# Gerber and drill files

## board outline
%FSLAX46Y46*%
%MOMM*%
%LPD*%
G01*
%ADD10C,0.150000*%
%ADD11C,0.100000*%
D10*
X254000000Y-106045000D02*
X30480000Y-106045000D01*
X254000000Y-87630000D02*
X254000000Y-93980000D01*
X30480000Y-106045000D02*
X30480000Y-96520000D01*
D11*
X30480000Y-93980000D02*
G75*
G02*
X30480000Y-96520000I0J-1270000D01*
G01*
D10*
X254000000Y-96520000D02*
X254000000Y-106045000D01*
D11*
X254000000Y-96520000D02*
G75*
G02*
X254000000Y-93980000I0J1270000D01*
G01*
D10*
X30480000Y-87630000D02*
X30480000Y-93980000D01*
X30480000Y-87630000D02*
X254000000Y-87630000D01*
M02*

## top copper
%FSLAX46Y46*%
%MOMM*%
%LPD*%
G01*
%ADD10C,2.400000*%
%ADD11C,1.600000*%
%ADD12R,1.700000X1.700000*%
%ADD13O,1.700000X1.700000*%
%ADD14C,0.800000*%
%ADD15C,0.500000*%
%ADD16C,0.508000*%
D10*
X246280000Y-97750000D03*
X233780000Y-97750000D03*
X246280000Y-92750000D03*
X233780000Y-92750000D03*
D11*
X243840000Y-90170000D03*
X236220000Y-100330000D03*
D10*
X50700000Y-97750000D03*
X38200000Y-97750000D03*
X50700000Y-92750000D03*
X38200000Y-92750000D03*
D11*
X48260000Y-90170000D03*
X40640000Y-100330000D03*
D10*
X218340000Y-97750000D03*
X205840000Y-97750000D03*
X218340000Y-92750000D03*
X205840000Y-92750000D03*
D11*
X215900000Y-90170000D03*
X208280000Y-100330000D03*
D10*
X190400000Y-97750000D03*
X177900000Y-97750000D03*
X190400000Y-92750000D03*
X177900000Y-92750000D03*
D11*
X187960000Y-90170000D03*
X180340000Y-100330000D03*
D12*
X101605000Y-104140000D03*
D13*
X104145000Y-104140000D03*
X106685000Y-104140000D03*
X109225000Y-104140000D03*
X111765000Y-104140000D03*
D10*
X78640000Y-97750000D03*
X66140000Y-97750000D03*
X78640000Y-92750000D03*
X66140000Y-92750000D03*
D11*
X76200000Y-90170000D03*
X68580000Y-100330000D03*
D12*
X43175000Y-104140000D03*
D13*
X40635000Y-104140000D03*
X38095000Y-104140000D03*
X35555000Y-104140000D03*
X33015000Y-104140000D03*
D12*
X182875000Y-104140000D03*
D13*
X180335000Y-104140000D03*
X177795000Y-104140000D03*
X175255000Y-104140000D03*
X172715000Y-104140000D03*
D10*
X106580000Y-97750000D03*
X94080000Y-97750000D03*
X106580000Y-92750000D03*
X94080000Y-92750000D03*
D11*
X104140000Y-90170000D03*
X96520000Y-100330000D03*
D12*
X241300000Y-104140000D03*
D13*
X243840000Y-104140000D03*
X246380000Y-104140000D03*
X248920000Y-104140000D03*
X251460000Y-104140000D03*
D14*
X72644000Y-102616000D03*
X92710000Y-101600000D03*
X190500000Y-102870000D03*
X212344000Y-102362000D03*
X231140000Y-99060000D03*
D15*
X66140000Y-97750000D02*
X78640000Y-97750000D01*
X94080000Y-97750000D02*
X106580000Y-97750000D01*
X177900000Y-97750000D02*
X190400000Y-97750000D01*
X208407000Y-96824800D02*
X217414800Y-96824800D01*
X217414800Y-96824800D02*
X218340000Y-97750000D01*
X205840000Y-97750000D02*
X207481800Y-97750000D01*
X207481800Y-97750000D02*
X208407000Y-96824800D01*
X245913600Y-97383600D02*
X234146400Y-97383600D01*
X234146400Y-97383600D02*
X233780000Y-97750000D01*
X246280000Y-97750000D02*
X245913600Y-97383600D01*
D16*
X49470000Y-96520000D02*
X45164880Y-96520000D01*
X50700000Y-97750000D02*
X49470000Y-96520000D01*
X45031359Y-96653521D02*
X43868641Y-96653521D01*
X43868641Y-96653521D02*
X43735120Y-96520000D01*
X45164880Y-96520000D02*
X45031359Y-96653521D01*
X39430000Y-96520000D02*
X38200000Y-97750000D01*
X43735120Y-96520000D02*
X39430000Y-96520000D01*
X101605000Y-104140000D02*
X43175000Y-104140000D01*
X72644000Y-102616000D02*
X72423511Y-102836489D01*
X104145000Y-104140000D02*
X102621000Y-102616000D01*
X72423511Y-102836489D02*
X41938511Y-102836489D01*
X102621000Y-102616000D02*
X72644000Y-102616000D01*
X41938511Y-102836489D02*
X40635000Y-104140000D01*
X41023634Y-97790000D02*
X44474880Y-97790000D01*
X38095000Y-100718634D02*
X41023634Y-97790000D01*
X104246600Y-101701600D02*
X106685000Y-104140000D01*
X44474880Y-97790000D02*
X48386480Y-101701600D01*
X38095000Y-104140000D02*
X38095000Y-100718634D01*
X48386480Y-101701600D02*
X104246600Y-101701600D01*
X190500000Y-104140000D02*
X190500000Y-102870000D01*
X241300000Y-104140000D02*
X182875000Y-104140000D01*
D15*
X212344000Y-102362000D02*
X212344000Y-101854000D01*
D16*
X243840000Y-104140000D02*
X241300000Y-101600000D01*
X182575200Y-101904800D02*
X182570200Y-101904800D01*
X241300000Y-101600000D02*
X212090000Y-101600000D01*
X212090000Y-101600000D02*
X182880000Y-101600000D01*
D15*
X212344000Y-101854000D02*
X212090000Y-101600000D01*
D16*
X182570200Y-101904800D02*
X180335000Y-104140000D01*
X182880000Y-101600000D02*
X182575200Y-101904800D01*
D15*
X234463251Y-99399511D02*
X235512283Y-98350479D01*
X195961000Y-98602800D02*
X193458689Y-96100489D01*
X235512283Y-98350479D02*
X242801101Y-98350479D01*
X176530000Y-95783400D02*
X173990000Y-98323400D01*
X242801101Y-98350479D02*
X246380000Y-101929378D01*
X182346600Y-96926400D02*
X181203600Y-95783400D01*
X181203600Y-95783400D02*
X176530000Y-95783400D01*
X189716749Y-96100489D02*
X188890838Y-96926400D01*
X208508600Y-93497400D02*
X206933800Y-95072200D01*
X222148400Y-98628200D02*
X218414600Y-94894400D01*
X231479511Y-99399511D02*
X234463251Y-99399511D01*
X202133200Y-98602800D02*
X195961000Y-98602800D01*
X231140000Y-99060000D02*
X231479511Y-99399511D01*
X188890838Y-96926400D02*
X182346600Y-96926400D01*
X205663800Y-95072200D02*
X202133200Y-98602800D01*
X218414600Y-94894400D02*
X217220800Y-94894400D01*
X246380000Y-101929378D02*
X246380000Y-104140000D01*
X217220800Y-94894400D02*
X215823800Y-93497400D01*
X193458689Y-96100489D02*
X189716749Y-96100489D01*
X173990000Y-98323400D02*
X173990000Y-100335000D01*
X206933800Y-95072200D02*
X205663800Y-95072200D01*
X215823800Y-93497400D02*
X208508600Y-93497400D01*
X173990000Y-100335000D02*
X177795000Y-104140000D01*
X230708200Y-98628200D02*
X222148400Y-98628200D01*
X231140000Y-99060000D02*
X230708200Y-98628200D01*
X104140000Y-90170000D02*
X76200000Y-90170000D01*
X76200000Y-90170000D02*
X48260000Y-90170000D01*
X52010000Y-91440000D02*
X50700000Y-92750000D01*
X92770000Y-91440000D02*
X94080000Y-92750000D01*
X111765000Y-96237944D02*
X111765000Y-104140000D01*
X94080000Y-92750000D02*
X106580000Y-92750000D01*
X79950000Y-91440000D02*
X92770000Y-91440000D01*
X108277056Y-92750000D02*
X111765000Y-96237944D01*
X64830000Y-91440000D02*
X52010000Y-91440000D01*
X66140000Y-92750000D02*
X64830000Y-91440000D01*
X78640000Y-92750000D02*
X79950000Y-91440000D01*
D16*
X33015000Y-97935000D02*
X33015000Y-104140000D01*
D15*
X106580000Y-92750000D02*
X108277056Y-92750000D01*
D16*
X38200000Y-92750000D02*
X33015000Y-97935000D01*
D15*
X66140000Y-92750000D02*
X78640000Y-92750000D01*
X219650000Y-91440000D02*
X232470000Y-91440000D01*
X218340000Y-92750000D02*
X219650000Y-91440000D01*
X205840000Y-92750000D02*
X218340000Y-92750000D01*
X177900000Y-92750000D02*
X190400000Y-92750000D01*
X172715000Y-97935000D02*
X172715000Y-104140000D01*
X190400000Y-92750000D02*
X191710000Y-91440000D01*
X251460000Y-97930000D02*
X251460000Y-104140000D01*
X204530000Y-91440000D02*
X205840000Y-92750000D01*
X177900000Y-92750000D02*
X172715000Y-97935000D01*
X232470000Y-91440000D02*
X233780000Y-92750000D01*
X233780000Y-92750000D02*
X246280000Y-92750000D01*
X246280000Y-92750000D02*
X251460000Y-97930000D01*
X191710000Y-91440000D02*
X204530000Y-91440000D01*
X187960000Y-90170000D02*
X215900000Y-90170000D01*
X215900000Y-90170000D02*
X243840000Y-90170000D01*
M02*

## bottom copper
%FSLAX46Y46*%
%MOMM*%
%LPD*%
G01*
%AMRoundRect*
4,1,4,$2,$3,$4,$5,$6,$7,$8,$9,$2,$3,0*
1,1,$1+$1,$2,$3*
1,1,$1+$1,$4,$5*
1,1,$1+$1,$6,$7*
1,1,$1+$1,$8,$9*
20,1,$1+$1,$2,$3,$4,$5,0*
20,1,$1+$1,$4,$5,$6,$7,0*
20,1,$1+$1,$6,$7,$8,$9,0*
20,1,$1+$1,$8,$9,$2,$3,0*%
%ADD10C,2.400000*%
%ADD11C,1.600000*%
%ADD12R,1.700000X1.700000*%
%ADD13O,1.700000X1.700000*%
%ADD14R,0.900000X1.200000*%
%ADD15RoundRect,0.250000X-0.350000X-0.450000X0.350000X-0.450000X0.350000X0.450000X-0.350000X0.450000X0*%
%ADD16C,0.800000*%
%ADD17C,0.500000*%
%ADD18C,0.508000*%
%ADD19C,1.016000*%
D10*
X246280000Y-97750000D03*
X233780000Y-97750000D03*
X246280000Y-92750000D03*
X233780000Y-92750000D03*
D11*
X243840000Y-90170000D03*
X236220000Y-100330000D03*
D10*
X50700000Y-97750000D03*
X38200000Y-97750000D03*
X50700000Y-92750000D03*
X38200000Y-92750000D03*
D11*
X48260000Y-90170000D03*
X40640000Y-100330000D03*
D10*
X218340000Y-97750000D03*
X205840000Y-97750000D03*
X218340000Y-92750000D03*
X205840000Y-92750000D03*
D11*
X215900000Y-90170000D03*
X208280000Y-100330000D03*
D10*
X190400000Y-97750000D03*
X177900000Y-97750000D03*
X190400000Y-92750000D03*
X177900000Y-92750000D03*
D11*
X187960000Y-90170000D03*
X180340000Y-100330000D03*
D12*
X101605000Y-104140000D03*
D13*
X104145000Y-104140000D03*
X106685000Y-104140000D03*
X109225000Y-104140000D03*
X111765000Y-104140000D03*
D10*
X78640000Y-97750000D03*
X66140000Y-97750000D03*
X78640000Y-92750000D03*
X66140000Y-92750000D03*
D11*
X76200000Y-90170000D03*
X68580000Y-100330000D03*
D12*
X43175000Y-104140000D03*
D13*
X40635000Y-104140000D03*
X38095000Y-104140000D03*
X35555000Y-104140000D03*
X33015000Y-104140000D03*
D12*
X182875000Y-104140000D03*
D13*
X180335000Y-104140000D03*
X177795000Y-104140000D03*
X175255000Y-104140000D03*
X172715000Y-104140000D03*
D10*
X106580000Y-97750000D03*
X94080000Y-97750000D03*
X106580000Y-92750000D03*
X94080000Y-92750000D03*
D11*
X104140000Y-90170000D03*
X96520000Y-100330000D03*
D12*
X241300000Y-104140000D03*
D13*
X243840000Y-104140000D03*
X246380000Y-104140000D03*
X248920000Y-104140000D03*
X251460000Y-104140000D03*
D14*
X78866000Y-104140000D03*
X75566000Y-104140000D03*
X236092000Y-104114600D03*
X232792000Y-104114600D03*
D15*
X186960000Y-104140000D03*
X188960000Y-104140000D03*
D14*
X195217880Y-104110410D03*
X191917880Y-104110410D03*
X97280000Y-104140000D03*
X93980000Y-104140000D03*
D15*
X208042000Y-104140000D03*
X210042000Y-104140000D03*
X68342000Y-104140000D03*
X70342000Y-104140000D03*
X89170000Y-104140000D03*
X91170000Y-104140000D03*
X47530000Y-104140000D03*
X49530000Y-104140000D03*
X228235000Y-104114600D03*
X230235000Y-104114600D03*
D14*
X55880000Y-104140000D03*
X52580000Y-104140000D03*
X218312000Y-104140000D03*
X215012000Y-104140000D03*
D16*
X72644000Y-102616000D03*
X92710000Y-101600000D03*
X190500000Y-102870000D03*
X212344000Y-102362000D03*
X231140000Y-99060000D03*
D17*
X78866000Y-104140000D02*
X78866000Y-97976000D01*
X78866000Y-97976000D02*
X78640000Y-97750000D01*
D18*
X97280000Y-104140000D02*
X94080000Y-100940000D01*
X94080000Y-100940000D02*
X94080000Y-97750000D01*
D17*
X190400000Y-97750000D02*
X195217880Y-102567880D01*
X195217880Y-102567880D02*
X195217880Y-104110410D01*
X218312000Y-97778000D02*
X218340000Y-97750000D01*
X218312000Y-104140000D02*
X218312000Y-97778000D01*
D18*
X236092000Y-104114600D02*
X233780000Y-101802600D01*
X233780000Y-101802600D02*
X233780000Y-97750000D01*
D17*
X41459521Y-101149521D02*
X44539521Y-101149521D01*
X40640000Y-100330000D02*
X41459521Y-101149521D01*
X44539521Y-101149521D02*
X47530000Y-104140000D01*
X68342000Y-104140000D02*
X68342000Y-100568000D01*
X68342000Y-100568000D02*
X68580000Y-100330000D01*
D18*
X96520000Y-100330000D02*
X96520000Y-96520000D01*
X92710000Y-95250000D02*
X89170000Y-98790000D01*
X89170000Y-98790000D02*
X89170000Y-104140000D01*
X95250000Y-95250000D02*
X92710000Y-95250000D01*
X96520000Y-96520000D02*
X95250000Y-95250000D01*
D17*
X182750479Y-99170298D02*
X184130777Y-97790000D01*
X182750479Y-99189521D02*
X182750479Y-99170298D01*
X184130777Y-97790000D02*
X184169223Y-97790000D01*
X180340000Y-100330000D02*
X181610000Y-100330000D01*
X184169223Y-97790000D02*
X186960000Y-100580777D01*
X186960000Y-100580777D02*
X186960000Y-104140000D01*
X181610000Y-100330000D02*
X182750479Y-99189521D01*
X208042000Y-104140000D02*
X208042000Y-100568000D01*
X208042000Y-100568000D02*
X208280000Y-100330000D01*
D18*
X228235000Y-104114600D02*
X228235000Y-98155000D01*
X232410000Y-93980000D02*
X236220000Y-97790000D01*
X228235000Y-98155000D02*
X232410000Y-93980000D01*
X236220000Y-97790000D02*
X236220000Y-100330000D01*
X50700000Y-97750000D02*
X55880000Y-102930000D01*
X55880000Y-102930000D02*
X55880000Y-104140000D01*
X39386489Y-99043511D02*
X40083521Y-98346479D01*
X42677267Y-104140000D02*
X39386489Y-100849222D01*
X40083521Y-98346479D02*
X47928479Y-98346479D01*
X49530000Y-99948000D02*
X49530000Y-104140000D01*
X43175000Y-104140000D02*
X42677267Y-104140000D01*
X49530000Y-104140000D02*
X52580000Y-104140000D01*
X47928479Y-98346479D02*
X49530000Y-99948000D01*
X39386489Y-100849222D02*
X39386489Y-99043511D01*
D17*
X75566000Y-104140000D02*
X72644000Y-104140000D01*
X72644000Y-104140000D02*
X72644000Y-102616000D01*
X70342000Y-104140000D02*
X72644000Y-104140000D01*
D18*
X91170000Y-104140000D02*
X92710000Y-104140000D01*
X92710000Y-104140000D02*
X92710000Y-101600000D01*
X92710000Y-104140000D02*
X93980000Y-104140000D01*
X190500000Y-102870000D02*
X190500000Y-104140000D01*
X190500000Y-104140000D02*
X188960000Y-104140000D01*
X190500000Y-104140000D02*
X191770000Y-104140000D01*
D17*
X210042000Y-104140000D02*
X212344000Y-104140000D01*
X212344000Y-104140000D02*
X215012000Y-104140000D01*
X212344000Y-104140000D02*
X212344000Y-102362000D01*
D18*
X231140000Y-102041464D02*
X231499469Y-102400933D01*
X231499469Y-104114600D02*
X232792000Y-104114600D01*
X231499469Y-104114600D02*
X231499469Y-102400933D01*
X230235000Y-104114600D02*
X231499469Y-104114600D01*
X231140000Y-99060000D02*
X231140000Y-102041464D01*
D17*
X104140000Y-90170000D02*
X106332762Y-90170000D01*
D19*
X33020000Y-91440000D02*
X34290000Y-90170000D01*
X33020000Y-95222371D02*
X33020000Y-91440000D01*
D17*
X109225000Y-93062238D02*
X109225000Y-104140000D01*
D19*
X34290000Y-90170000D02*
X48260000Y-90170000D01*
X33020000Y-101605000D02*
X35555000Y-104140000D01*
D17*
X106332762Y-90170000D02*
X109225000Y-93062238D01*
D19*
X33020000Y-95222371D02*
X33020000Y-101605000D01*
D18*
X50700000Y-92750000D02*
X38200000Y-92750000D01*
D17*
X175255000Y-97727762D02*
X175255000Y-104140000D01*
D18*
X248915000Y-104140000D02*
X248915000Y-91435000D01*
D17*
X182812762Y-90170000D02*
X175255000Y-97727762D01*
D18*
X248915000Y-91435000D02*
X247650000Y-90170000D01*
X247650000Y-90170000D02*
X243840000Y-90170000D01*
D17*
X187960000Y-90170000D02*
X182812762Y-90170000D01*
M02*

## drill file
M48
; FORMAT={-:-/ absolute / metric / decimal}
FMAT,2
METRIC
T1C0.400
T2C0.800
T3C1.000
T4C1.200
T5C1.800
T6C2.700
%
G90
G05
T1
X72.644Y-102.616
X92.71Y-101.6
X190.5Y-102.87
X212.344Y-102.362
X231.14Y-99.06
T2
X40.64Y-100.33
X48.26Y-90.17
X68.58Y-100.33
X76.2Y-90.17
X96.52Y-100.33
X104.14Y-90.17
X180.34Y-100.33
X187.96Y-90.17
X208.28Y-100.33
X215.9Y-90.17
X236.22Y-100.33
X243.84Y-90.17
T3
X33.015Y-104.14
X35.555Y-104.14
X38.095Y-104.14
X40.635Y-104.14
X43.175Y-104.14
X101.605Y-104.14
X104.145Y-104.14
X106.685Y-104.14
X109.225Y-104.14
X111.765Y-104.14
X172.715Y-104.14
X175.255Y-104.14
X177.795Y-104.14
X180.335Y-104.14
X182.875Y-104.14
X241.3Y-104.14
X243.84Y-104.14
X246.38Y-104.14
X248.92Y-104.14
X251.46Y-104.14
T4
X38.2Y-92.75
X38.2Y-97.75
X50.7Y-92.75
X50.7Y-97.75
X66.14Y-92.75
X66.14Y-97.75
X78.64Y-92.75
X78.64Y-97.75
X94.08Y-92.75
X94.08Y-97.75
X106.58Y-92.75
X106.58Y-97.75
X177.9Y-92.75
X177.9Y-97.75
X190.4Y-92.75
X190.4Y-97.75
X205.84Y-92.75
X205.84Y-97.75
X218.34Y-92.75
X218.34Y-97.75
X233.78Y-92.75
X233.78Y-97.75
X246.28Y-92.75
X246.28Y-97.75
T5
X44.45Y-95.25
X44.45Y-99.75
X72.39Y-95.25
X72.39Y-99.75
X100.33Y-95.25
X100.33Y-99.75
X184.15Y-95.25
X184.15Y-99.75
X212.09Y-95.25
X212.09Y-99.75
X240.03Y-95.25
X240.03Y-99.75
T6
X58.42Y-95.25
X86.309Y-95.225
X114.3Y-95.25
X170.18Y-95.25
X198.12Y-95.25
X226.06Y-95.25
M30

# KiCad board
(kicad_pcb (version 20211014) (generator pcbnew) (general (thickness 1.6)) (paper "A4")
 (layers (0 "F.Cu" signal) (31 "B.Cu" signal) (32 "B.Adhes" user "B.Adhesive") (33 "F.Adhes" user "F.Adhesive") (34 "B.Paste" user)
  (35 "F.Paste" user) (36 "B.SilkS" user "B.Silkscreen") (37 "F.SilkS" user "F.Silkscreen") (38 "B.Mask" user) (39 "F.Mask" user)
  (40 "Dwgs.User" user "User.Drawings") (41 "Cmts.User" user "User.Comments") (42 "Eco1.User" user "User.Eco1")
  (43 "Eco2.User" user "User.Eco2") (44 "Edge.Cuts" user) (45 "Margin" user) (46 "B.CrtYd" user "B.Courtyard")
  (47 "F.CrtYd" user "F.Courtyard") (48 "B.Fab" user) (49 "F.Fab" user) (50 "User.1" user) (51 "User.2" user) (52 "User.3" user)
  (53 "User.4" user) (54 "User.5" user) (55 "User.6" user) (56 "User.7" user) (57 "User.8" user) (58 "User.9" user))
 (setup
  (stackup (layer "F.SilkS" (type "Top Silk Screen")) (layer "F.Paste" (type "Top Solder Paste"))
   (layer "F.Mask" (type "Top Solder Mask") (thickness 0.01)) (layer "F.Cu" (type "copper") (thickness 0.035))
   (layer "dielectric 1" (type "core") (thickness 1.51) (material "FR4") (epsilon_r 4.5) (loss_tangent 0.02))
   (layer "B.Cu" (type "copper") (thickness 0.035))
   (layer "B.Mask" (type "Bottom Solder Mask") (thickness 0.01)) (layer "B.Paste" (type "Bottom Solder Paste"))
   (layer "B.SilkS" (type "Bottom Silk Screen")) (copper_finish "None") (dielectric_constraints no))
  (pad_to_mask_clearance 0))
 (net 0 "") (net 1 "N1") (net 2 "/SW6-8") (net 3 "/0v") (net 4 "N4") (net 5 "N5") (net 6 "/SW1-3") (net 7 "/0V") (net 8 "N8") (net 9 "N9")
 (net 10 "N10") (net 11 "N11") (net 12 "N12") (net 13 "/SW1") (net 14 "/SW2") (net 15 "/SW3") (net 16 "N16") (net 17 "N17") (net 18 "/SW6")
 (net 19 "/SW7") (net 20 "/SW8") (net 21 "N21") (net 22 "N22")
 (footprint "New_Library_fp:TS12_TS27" (layer "F.Cu") (at 240.03 95.25 180)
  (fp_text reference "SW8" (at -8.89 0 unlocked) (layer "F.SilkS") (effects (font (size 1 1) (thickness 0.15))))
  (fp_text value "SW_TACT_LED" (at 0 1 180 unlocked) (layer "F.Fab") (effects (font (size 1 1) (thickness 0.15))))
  (pad "" np_thru_hole circle (at 0 -4.5 180) (size 1.8 1.8) (drill 1.8) (layers *.Mask) (zone_connect 0))
  (pad "" np_thru_hole circle (at 0 0 180) (size 1.8 1.8) (drill 1.8) (layers *.Mask) (zone_connect 0))
  (pad "1" thru_hole circle (at -6.25 -2.5 180) (size 2.4 2.4) (drill 1.2) (layers *.Cu *.Mask) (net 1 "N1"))
  (pad "2" thru_hole circle (at 6.25 -2.5 180) (size 2.4 2.4) (drill 1.2) (layers *.Cu *.Mask) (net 1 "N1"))
  (pad "3" thru_hole circle (at -6.25 2.5 180) (size 2.4 2.4) (drill 1.2) (layers *.Cu *.Mask) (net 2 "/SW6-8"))
  (pad "4" thru_hole circle (at 6.25 2.5 180) (size 2.4 2.4) (drill 1.2) (layers *.Cu *.Mask) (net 2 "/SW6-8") (zone_connect 2))
  (pad "5" thru_hole circle (at -3.81 5.08 180) (size 1.6 1.6) (drill 0.8) (layers *.Cu *.Mask) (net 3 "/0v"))
  (pad "6" thru_hole circle (at 3.81 -5.08 180) (size 1.6 1.6) (drill 0.8) (layers *.Cu *.Mask) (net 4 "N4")))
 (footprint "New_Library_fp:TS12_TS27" (layer "F.Cu") (at 44.45 95.25 180)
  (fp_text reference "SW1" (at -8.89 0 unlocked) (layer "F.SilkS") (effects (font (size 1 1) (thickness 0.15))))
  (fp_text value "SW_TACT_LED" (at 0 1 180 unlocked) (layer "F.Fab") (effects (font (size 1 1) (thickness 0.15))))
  (pad "" np_thru_hole circle (at 0 -4.5 180) (size 1.8 1.8) (drill 1.8) (layers *.Mask) (zone_connect 0))
  (pad "" np_thru_hole circle (at 0 0 180) (size 1.8 1.8) (drill 1.8) (layers *.Mask) (zone_connect 0))
  (pad "1" thru_hole circle (at -6.25 -2.5 180) (size 2.4 2.4) (drill 1.2) (layers *.Cu *.Mask) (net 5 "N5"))
  (pad "2" thru_hole circle (at 6.25 -2.5 180) (size 2.4 2.4) (drill 1.2) (layers *.Cu *.Mask) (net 5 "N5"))
  (pad "3" thru_hole circle (at -6.25 2.5 180) (size 2.4 2.4) (drill 1.2) (layers *.Cu *.Mask) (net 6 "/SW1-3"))
  (pad "4" thru_hole circle (at 6.25 2.5 180) (size 2.4 2.4) (drill 1.2) (layers *.Cu *.Mask) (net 6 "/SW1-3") (zone_connect 2))
  (pad "5" thru_hole circle (at -3.81 5.08 180) (size 1.6 1.6) (drill 0.8) (layers *.Cu *.Mask) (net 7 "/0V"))
  (pad "6" thru_hole circle (at 3.81 -5.08 180) (size 1.6 1.6) (drill 0.8) (layers *.Cu *.Mask) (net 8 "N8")))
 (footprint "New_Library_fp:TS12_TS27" (layer "F.Cu") (at 212.09 95.25 180)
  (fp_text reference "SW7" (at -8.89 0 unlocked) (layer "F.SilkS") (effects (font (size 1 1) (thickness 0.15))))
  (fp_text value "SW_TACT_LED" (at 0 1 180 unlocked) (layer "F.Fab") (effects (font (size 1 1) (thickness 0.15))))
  (pad "" np_thru_hole circle (at 0 -4.5 180) (size 1.8 1.8) (drill 1.8) (layers *.Mask) (zone_connect 0))
  (pad "" np_thru_hole circle (at 0 0 180) (size 1.8 1.8) (drill 1.8) (layers *.Mask) (zone_connect 0))
  (pad "1" thru_hole circle (at -6.25 -2.5 180) (size 2.4 2.4) (drill 1.2) (layers *.Cu *.Mask) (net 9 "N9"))
  (pad "2" thru_hole circle (at 6.25 -2.5 180) (size 2.4 2.4) (drill 1.2) (layers *.Cu *.Mask) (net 9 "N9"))
  (pad "3" thru_hole circle (at -6.25 2.5 180) (size 2.4 2.4) (drill 1.2) (layers *.Cu *.Mask) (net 2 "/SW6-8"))
  (pad "4" thru_hole circle (at 6.25 2.5 180) (size 2.4 2.4) (drill 1.2) (layers *.Cu *.Mask) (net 2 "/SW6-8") (zone_connect 2))
  (pad "5" thru_hole circle (at -3.81 5.08 180) (size 1.6 1.6) (drill 0.8) (layers *.Cu *.Mask) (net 3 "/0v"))
  (pad "6" thru_hole circle (at 3.81 -5.08 180) (size 1.6 1.6) (drill 0.8) (layers *.Cu *.Mask) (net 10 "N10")))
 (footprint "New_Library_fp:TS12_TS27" (layer "F.Cu") (at 184.15 95.25 180)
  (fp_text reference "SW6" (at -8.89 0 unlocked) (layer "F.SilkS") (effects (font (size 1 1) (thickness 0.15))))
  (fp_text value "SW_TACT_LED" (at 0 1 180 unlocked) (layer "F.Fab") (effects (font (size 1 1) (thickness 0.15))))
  (pad "" np_thru_hole circle (at 0 -4.5 180) (size 1.8 1.8) (drill 1.8) (layers *.Mask) (zone_connect 0))
  (pad "" np_thru_hole circle (at 0 0 180) (size 1.8 1.8) (drill 1.8) (layers *.Mask) (zone_connect 0))
  (pad "1" thru_hole circle (at -6.25 -2.5 180) (size 2.4 2.4) (drill 1.2) (layers *.Cu *.Mask) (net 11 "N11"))
  (pad "2" thru_hole circle (at 6.25 -2.5 180) (size 2.4 2.4) (drill 1.2) (layers *.Cu *.Mask) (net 11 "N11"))
  (pad "3" thru_hole circle (at -6.25 2.5 180) (size 2.4 2.4) (drill 1.2) (layers *.Cu *.Mask) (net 2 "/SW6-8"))
  (pad "4" thru_hole circle (at 6.25 2.5 180) (size 2.4 2.4) (drill 1.2) (layers *.Cu *.Mask) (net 2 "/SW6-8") (zone_connect 2))
  (pad "5" thru_hole circle (at -3.81 5.08 180) (size 1.6 1.6) (drill 0.8) (layers *.Cu *.Mask) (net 3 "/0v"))
  (pad "6" thru_hole circle (at 3.81 -5.08 180) (size 1.6 1.6) (drill 0.8) (layers *.Cu *.Mask) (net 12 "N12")))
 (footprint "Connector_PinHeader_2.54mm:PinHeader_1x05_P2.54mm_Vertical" (layer "F.Cu") (at 101.605 104.14 90)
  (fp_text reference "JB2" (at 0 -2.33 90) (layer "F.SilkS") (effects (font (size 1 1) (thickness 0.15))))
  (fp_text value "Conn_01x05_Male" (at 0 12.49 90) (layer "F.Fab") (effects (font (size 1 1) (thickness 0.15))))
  (pad "1" thru_hole rect (at 0 0 90) (size 1.7 1.7) (drill 1) (layers *.Cu *.Mask) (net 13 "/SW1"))
  (pad "2" thru_hole oval (at 0 2.54 90) (size 1.7 1.7) (drill 1) (layers *.Cu *.Mask) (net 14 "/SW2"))
  (pad "3" thru_hole oval (at 0 5.08 90) (size 1.7 1.7) (drill 1) (layers *.Cu *.Mask) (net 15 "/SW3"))
  (pad "4" thru_hole oval (at 0 7.62 90) (size 1.7 1.7) (drill 1) (layers *.Cu *.Mask) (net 7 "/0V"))
  (pad "5" thru_hole oval (at 0 10.16 90) (size 1.7 1.7) (drill 1) (layers *.Cu *.Mask) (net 6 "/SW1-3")))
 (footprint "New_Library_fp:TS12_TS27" (layer "F.Cu") (at 72.39 95.25 180)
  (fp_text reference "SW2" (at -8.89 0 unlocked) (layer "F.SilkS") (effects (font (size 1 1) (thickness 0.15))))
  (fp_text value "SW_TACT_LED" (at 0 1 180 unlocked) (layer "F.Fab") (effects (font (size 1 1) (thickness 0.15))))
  (pad "" np_thru_hole circle (at 0 0 180) (size 1.8 1.8) (drill 1.8) (layers *.Mask) (zone_connect 0))
  (pad "" np_thru_hole circle (at 0 -4.5 180) (size 1.8 1.8) (drill 1.8) (layers *.Mask) (zone_connect 0))
  (pad "1" thru_hole circle (at -6.25 -2.5 180) (size 2.4 2.4) (drill 1.2) (layers *.Cu *.Mask) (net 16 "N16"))
  (pad "2" thru_hole circle (at 6.25 -2.5 180) (size 2.4 2.4) (drill 1.2) (layers *.Cu *.Mask) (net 16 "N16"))
  (pad "3" thru_hole circle (at -6.25 2.5 180) (size 2.4 2.4) (drill 1.2) (layers *.Cu *.Mask) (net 6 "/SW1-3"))
  (pad "4" thru_hole circle (at 6.25 2.5 180) (size 2.4 2.4) (drill 1.2) (layers *.Cu *.Mask) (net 6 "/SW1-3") (zone_connect 2))
  (pad "5" thru_hole circle (at -3.81 5.08 180) (size 1.6 1.6) (drill 0.8) (layers *.Cu *.Mask) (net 7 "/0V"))
  (pad "6" thru_hole circle (at 3.81 -5.08 180) (size 1.6 1.6) (drill 0.8) (layers *.Cu *.Mask) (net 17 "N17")))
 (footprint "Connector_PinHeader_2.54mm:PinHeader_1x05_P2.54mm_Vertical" (layer "F.Cu") (at 43.175 104.14 -90)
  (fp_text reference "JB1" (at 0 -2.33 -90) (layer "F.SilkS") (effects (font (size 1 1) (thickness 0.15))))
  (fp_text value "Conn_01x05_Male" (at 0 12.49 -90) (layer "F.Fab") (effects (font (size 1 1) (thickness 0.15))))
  (pad "1" thru_hole rect (at 0 0 270) (size 1.7 1.7) (drill 1) (layers *.Cu *.Mask) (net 13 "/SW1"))
  (pad "2" thru_hole oval (at 0 2.54 270) (size 1.7 1.7) (drill 1) (layers *.Cu *.Mask) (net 14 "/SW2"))
  (pad "3" thru_hole oval (at 0 5.08 270) (size 1.7 1.7) (drill 1) (layers *.Cu *.Mask) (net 15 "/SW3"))
  (pad "4" thru_hole oval (at 0 7.62 270) (size 1.7 1.7) (drill 1) (layers *.Cu *.Mask) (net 7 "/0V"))
  (pad "5" thru_hole oval (at 0 10.16 270) (size 1.7 1.7) (drill 1) (layers *.Cu *.Mask) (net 6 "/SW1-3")))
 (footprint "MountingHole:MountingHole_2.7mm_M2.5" (layer "F.Cu") (at 86.3092 95.2246 90)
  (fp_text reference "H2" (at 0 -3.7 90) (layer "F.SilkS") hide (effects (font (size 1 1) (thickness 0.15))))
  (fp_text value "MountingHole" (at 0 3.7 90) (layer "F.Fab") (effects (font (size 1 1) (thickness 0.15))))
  (pad "" np_thru_hole circle (at 0 0 90) (size 2.7 2.7) (drill 2.7) (layers *.Cu *.Mask)))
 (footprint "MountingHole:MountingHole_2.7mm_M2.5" (layer "F.Cu") (at 114.3 95.25 90)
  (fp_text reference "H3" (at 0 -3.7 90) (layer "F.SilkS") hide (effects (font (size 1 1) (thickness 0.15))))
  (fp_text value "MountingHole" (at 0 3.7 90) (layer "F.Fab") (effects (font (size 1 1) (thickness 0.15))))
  (pad "" np_thru_hole circle (at 0 0 90) (size 2.7 2.7) (drill 2.7) (layers *.Cu *.Mask)))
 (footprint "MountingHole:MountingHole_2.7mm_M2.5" (layer "F.Cu") (at 58.42 95.25 90)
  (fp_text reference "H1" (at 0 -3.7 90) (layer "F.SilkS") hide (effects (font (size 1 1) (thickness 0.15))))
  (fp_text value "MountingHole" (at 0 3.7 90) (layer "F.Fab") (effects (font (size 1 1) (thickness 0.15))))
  (pad "" np_thru_hole circle (at 0 0 90) (size 2.7 2.7) (drill 2.7) (layers *.Cu *.Mask)))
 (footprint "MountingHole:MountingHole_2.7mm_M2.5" (layer "F.Cu") (at 226.06 95.25 90)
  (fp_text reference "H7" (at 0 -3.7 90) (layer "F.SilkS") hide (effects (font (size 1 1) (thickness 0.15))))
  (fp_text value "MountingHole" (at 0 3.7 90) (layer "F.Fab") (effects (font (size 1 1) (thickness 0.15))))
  (pad "" np_thru_hole circle (at 0 0 90) (size 2.7 2.7) (drill 2.7) (layers *.Cu *.Mask)))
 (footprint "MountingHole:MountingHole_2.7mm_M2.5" (layer "F.Cu") (at 198.12 95.25 90)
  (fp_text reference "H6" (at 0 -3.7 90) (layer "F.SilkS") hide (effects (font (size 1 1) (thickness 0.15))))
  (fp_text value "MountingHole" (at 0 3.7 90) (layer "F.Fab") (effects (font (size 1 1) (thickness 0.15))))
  (pad "" np_thru_hole circle (at 0 0 90) (size 2.7 2.7) (drill 2.7) (layers *.Cu *.Mask)))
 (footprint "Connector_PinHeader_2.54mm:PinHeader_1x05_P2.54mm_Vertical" (layer "F.Cu") (at 182.875 104.14 -90)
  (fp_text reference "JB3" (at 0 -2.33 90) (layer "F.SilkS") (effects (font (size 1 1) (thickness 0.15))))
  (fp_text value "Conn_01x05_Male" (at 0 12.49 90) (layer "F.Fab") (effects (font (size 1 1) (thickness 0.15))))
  (pad "1" thru_hole rect (at 0 0 270) (size 1.7 1.7) (drill 1) (layers *.Cu *.Mask) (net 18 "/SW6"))
  (pad "2" thru_hole oval (at 0 2.54 270) (size 1.7 1.7) (drill 1) (layers *.Cu *.Mask) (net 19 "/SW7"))
  (pad "3" thru_hole oval (at 0 5.08 270) (size 1.7 1.7) (drill 1) (layers *.Cu *.Mask) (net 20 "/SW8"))
  (pad "4" thru_hole oval (at 0 7.62 270) (size 1.7 1.7) (drill 1) (layers *.Cu *.Mask) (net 3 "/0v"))
  (pad "5" thru_hole oval (at 0 10.16 270) (size 1.7 1.7) (drill 1) (layers *.Cu *.Mask) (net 2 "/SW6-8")))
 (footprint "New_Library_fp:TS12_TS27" (layer "F.Cu") (at 100.33 95.25 180)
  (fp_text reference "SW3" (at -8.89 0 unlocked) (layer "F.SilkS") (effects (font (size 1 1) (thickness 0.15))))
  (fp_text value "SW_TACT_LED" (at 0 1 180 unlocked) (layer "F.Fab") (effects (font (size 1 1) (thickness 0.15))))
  (pad "" np_thru_hole circle (at 0 -4.5 180) (size 1.8 1.8) (drill 1.8) (layers *.Mask) (zone_connect 0))
  (pad "" np_thru_hole circle (at 0 0 180) (size 1.8 1.8) (drill 1.8) (layers *.Mask) (zone_connect 0))
  (pad "1" thru_hole circle (at -6.25 -2.5 180) (size 2.4 2.4) (drill 1.2) (layers *.Cu *.Mask) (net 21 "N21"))
  (pad "2" thru_hole circle (at 6.25 -2.5 180) (size 2.4 2.4) (drill 1.2) (layers *.Cu *.Mask) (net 21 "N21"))
  (pad "3" thru_hole circle (at -6.25 2.5 180) (size 2.4 2.4) (drill 1.2) (layers *.Cu *.Mask) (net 6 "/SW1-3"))
  (pad "4" thru_hole circle (at 6.25 2.5 180) (size 2.4 2.4) (drill 1.2) (layers *.Cu *.Mask) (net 6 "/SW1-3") (zone_connect 2))
  (pad "5" thru_hole circle (at -3.81 5.08 180) (size 1.6 1.6) (drill 0.8) (layers *.Cu *.Mask) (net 7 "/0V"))
  (pad "6" thru_hole circle (at 3.81 -5.08 180) (size 1.6 1.6) (drill 0.8) (layers *.Cu *.Mask) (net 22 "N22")))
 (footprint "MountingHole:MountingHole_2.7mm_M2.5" (layer "F.Cu") (at 170.18 95.25 90)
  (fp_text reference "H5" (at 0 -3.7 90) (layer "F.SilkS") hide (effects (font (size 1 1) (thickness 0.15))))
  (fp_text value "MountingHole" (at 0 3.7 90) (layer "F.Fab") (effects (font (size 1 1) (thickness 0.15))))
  (pad "" np_thru_hole circle (at 0 0 90) (size 2.7 2.7) (drill 2.7) (layers *.Cu *.Mask)))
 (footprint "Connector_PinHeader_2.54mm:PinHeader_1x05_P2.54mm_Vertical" (layer "F.Cu") (at 241.3 104.14 90)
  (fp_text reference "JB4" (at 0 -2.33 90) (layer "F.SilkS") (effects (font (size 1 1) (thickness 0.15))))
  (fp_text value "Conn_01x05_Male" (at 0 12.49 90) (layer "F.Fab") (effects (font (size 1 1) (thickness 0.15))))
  (pad "1" thru_hole rect (at 0 0 90) (size 1.7 1.7) (drill 1) (layers *.Cu *.Mask) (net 18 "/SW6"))
  (pad "2" thru_hole oval (at 0 2.54 90) (size 1.7 1.7) (drill 1) (layers *.Cu *.Mask) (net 19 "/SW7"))
  (pad "3" thru_hole oval (at 0 5.08 90) (size 1.7 1.7) (drill 1) (layers *.Cu *.Mask) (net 20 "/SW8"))
  (pad "4" thru_hole oval (at 0 7.62 90) (size 1.7 1.7) (drill 1) (layers *.Cu *.Mask) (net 3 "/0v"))
  (pad "5" thru_hole oval (at 0 10.16 90) (size 1.7 1.7) (drill 1) (layers *.Cu *.Mask) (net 2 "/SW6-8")))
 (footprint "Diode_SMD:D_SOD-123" (layer "B.Cu") (at 77.216 104.14 180)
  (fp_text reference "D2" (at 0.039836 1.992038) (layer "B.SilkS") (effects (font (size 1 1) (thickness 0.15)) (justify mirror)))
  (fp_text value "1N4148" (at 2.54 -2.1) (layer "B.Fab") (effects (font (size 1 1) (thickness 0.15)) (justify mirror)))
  (pad "1" smd rect (at -1.65 0 180) (size 0.9 1.2) (layers "B.Cu" "B.Paste" "B.Mask") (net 16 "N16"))
  (pad "2" smd rect (at 1.65 0 180) (size 0.9 1.2) (layers "B.Cu" "B.Paste" "B.Mask") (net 14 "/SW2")))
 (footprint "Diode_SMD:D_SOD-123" (layer "B.Cu") (at 234.442 104.1146 180)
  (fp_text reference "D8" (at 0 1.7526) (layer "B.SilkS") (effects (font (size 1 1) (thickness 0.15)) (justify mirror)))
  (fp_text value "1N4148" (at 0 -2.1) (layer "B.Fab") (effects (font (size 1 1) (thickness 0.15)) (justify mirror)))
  (pad "1" smd rect (at -1.65 0 180) (size 0.9 1.2) (layers "B.Cu" "B.Paste" "B.Mask") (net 1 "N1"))
  (pad "2" smd rect (at 1.65 0 180) (size 0.9 1.2) (layers "B.Cu" "B.Paste" "B.Mask") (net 20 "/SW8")))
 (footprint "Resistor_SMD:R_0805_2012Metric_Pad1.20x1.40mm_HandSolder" (layer "B.Cu") (at 187.96 104.14)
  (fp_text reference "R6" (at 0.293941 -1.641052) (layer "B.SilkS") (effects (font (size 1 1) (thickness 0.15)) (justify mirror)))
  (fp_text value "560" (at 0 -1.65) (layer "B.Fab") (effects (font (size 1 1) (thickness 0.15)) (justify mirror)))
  (pad "1" smd roundrect (at -1 0) (size 1.2 1.4) (layers "B.Cu" "B.Paste" "B.Mask") (roundrect_rratio 0.2083333333) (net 12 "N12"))
  (pad "2" smd roundrect (at 1 0) (size 1.2 1.4) (layers "B.Cu" "B.Paste" "B.Mask") (roundrect_rratio 0.2083333333) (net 18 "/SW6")))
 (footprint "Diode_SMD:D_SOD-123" (layer "B.Cu") (at 193.56788 104.11041 180)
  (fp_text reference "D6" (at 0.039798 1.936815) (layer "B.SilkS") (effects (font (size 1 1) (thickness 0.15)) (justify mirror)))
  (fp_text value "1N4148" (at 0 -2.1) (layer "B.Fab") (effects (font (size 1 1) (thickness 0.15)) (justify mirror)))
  (pad "1" smd rect (at -1.65 0 180) (size 0.9 1.2) (layers "B.Cu" "B.Paste" "B.Mask") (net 11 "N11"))
  (pad "2" smd rect (at 1.65 0 180) (size 0.9 1.2) (layers "B.Cu" "B.Paste" "B.Mask") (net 18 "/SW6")))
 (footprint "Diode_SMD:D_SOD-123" (layer "B.Cu") (at 95.63 104.14 180)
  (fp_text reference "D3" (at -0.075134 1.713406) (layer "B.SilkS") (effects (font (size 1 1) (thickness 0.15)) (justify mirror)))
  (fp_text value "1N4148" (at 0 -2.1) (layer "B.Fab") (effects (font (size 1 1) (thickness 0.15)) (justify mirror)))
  (pad "1" smd rect (at -1.65 0 180) (size 0.9 1.2) (layers "B.Cu" "B.Paste" "B.Mask") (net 21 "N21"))
  (pad "2" smd rect (at 1.65 0 180) (size 0.9 1.2) (layers "B.Cu" "B.Paste" "B.Mask") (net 15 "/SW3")))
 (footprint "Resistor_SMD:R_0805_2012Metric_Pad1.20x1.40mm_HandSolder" (layer "B.Cu") (at 209.042 104.14)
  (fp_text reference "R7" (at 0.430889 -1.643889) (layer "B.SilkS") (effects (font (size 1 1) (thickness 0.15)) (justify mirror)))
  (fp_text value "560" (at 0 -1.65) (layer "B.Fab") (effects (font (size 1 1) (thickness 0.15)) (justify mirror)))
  (pad "1" smd roundrect (at -1 0) (size 1.2 1.4) (layers "B.Cu" "B.Paste" "B.Mask") (roundrect_rratio 0.2083333333) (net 10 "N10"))
  (pad "2" smd roundrect (at 1 0) (size 1.2 1.4) (layers "B.Cu" "B.Paste" "B.Mask") (roundrect_rratio 0.2083333333) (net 19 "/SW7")))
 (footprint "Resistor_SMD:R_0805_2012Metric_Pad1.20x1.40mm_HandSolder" (layer "B.Cu") (at 69.342 104.14)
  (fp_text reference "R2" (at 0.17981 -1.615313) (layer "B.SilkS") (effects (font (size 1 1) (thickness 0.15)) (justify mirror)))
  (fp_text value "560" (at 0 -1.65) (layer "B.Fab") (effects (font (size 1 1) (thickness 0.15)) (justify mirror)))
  (pad "1" smd roundrect (at -1 0) (size 1.2 1.4) (layers "B.Cu" "B.Paste" "B.Mask") (roundrect_rratio 0.2083333333) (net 17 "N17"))
  (pad "2" smd roundrect (at 1 0) (size 1.2 1.4) (layers "B.Cu" "B.Paste" "B.Mask") (roundrect_rratio 0.2083333333) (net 14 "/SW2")))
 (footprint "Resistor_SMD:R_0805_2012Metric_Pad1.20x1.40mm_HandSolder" (layer "B.Cu") (at 90.17 104.14)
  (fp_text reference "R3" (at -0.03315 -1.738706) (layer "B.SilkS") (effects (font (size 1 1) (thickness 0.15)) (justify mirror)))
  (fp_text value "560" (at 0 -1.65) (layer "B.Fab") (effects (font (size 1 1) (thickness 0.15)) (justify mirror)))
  (pad "1" smd roundrect (at -1 0) (size 1.2 1.4) (layers "B.Cu" "B.Paste" "B.Mask") (roundrect_rratio 0.2083333333) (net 22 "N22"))
  (pad "2" smd roundrect (at 1 0) (size 1.2 1.4) (layers "B.Cu" "B.Paste" "B.Mask") (roundrect_rratio 0.2083333333) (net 15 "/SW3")))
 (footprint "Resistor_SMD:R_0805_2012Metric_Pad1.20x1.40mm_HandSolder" (layer "B.Cu") (at 48.53 104.14)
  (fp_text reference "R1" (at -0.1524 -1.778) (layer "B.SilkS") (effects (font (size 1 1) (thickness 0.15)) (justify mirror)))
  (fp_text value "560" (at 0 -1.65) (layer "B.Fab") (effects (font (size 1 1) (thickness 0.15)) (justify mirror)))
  (pad "1" smd roundrect (at -1 0) (size 1.2 1.4) (layers "B.Cu" "B.Paste" "B.Mask") (roundrect_rratio 0.2083333333) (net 8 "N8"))
  (pad "2" smd roundrect (at 1 0) (size 1.2 1.4) (layers "B.Cu" "B.Paste" "B.Mask") (roundrect_rratio 0.2083333333) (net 13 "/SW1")))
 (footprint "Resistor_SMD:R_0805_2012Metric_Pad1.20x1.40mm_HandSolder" (layer "B.Cu") (at 229.235 104.1146)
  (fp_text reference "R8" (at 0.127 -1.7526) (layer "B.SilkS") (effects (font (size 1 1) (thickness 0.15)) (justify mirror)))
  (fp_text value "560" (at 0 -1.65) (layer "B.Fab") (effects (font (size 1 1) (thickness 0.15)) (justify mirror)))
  (pad "1" smd roundrect (at -1 0) (size 1.2 1.4) (layers "B.Cu" "B.Paste" "B.Mask") (roundrect_rratio 0.2083333333) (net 4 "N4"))
  (pad "2" smd roundrect (at 1 0) (size 1.2 1.4) (layers "B.Cu" "B.Paste" "B.Mask") (roundrect_rratio 0.2083333333) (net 20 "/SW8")))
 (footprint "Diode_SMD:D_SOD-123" (layer "B.Cu") (at 54.23 104.14 180)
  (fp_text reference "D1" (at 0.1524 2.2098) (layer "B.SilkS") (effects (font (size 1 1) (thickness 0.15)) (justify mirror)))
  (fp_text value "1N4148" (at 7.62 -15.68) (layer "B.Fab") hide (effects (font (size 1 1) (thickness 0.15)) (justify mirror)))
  (pad "1" smd rect (at -1.65 0 180) (size 0.9 1.2) (layers "B.Cu" "B.Paste" "B.Mask") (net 5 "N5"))
  (pad "2" smd rect (at 1.65 0 180) (size 0.9 1.2) (layers "B.Cu" "B.Paste" "B.Mask") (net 13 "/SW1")))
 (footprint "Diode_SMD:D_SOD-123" (layer "B.Cu") (at 216.662 104.14 180)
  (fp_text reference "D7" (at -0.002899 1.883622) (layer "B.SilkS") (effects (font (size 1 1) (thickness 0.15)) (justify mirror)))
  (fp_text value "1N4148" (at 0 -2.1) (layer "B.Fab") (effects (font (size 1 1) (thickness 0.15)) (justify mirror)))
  (pad "1" smd rect (at -1.65 0 180) (size 0.9 1.2) (layers "B.Cu" "B.Paste" "B.Mask") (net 9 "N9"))
  (pad "2" smd rect (at 1.65 0 180) (size 0.9 1.2) (layers "B.Cu" "B.Paste" "B.Mask") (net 19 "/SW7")))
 (gr_line (start 254 106.045) (end 30.48 106.045) (layer "Edge.Cuts") (width 0.15))
 (gr_line (start 254 87.63) (end 254 93.98) (layer "Edge.Cuts") (width 0.15))
 (gr_line (start 30.48 106.045) (end 30.48 96.52) (layer "Edge.Cuts") (width 0.15))
 (gr_arc (start 30.48 93.98) (mid 31.75 95.25) (end 30.48 96.52) (layer "Edge.Cuts") (width 0.1))
 (gr_line (start 254 96.52) (end 254 106.045) (layer "Edge.Cuts") (width 0.15))
 (gr_arc (start 254 96.52) (mid 252.73 95.25) (end 254 93.98) (layer "Edge.Cuts") (width 0.1))
 (gr_line (start 30.48 87.63) (end 30.48 93.98) (layer "Edge.Cuts") (width 0.15))
 (gr_line (start 30.48 87.63) (end 254 87.63) (layer "Edge.Cuts") (width 0.15))
 (segment (start 66.14 97.75) (end 78.64 97.75) (width 0.5) (layer "F.Cu") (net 16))
 (segment (start 78.866 104.14) (end 78.866 97.976) (width 0.5) (layer "B.Cu") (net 16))
 (segment (start 78.866 97.976) (end 78.64 97.75) (width 0.5) (layer "B.Cu") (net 16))
 (segment (start 94.08 97.75) (end 106.58 97.75) (width 0.5) (layer "F.Cu") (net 21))
 (segment (start 97.28 104.14) (end 94.08 100.94) (width 0.508) (layer "B.Cu") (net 21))
 (segment (start 94.08 100.94) (end 94.08 97.75) (width 0.508) (layer "B.Cu") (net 21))
 (segment (start 177.9 97.75) (end 190.4 97.75) (width 0.5) (layer "F.Cu") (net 11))
 (segment (start 190.4 97.75) (end 195.21788 102.56788) (width 0.5) (layer "B.Cu") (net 11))
 (segment (start 195.21788 102.56788) (end 195.21788 104.11041) (width 0.5) (layer "B.Cu") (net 11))
 (segment (start 208.407 96.8248) (end 217.4148 96.8248) (width 0.5) (layer "F.Cu") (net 9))
 (segment (start 217.4148 96.8248) (end 218.34 97.75) (width 0.5) (layer "F.Cu") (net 9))
 (segment (start 205.84 97.75) (end 207.4818 97.75) (width 0.5) (layer "F.Cu") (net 9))
 (segment (start 207.4818 97.75) (end 208.407 96.8248) (width 0.5) (layer "F.Cu") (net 9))
 (segment (start 218.312 97.778) (end 218.34 97.75) (width 0.5) (layer "B.Cu") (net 9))
 (segment (start 218.312 104.14) (end 218.312 97.778) (width 0.5) (layer "B.Cu") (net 9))
 (segment (start 245.9136 97.3836) (end 234.1464 97.3836) (width 0.5) (layer "F.Cu") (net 1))
 (segment (start 234.1464 97.3836) (end 233.78 97.75) (width 0.5) (layer "F.Cu") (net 1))
 (segment (start 246.28 97.75) (end 245.9136 97.3836) (width 0.5) (layer "F.Cu") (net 1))
 (segment (start 236.092 104.1146) (end 233.78 101.8026) (width 0.508) (layer "B.Cu") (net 1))
 (segment (start 233.78 101.8026) (end 233.78 97.75) (width 0.508) (layer "B.Cu") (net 1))
 (segment (start 41.459521 101.149521) (end 44.539521 101.149521) (width 0.5) (layer "B.Cu") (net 8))
 (segment (start 40.64 100.33) (end 41.459521 101.149521) (width 0.5) (layer "B.Cu") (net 8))
 (segment (start 44.539521 101.149521) (end 47.53 104.14) (width 0.5) (layer "B.Cu") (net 8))
 (segment (start 68.342 104.14) (end 68.342 100.568) (width 0.5) (layer "B.Cu") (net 17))
 (segment (start 68.342 100.568) (end 68.58 100.33) (width 0.5) (layer "B.Cu") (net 17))
 (segment (start 96.52 100.33) (end 96.52 96.52) (width 0.508) (layer "B.Cu") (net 22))
 (segment (start 92.71 95.25) (end 89.17 98.79) (width 0.508) (layer "B.Cu") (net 22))
 (segment (start 89.17 98.79) (end 89.17 104.14) (width 0.508) (layer "B.Cu") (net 22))
 (segment (start 95.25 95.25) (end 92.71 95.25) (width 0.508) (layer "B.Cu") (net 22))
 (segment (start 96.52 96.52) (end 95.25 95.25) (width 0.508) (layer "B.Cu") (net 22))
 (segment (start 182.750479 99.170298) (end 184.130777 97.79) (width 0.5) (layer "B.Cu") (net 12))
 (segment (start 182.750479 99.189521) (end 182.750479 99.170298) (width 0.5) (layer "B.Cu") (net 12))
 (segment (start 184.130777 97.79) (end 184.169223 97.79) (width 0.5) (layer "B.Cu") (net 12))
 (segment (start 180.34 100.33) (end 181.61 100.33) (width 0.5) (layer "B.Cu") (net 12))
 (segment (start 184.169223 97.79) (end 186.96 100.580777) (width 0.5) (layer "B.Cu") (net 12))
 (segment (start 186.96 100.580777) (end 186.96 104.14) (width 0.5) (layer "B.Cu") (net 12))
 (segment (start 181.61 100.33) (end 182.750479 99.189521) (width 0.5) (layer "B.Cu") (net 12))
 (segment (start 208.042 104.14) (end 208.042 100.568) (width 0.5) (layer "B.Cu") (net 10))
 (segment (start 208.042 100.568) (end 208.28 100.33) (width 0.5) (layer "B.Cu") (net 10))
 (segment (start 228.235 104.1146) (end 228.235 98.155) (width 0.508) (layer "B.Cu") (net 4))
 (segment (start 232.41 93.98) (end 236.22 97.79) (width 0.508) (layer "B.Cu") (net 4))
 (segment (start 228.235 98.155) (end 232.41 93.98) (width 0.508) (layer "B.Cu") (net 4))
 (segment (start 236.22 97.79) (end 236.22 100.33) (width 0.508) (layer "B.Cu") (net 4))
 (segment (start 49.47 96.52) (end 45.16488 96.52) (width 0.508) (layer "F.Cu") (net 5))
 (segment (start 50.7 97.75) (end 49.47 96.52) (width 0.508) (layer "F.Cu") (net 5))
 (segment (start 45.031359 96.653521) (end 43.868641 96.653521) (width 0.508) (layer "F.Cu") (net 5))
 (segment (start 43.868641 96.653521) (end 43.73512 96.52) (width 0.508) (layer "F.Cu") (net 5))
 (segment (start 45.16488 96.52) (end 45.031359 96.653521) (width 0.508) (layer "F.Cu") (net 5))
 (segment (start 39.43 96.52) (end 38.2 97.75) (width 0.508) (layer "F.Cu") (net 5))
 (segment (start 43.73512 96.52) (end 39.43 96.52) (width 0.508) (layer "F.Cu") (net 5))
 (segment (start 50.7 97.75) (end 55.88 102.93) (width 0.508) (layer "B.Cu") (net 5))
 (segment (start 55.88 102.93) (end 55.88 104.14) (width 0.508) (layer "B.Cu") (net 5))
 (segment (start 101.605 104.14) (end 43.175 104.14) (width 0.508) (layer "F.Cu") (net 13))
 (segment (start 39.386489 99.043511) (end 40.083521 98.346479) (width 0.508) (layer "B.Cu") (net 13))
 (segment (start 42.677267 104.14) (end 39.386489 100.849222) (width 0.508) (layer "B.Cu") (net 13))
 (segment (start 40.083521 98.346479) (end 47.928479 98.346479) (width 0.508) (layer "B.Cu") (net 13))
 (segment (start 49.53 99.948) (end 49.53 104.14) (width 0.508) (layer "B.Cu") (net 13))
 (segment (start 43.175 104.14) (end 42.677267 104.14) (width 0.508) (layer "B.Cu") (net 13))
 (segment (start 49.53 104.14) (end 52.58 104.14) (width 0.508) (layer "B.Cu") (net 13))
 (segment (start 47.928479 98.346479) (end 49.53 99.948) (width 0.508) (layer "B.Cu") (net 13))
 (segment (start 39.386489 100.849222) (end 39.386489 99.043511) (width 0.508) (layer "B.Cu") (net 13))
 (segment (start 72.644 102.616) (end 72.423511 102.836489) (width 0.508) (layer "F.Cu") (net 14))
 (segment (start 104.145 104.14) (end 102.621 102.616) (width 0.508) (layer "F.Cu") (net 14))
 (segment (start 72.423511 102.836489) (end 41.938511 102.836489) (width 0.508) (layer "F.Cu") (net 14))
 (segment (start 102.621 102.616) (end 72.644 102.616) (width 0.508) (layer "F.Cu") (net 14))
 (segment (start 41.938511 102.836489) (end 40.635 104.14) (width 0.508) (layer "F.Cu") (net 14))
 (via (at 72.644 102.616) (size 0.8) (drill 0.4) (layers "F.Cu" "B.Cu") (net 14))
 (segment (start 75.566 104.14) (end 72.644 104.14) (width 0.5) (layer "B.Cu") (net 14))
 (segment (start 72.644 104.14) (end 72.644 102.616) (width 0.5) (layer "B.Cu") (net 14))
 (segment (start 70.342 104.14) (end 72.644 104.14) (width 0.5) (layer "B.Cu") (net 14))
 (segment (start 41.023634 97.79) (end 44.47488 97.79) (width 0.508) (layer "F.Cu") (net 15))
 (segment (start 38.095 100.718634) (end 41.023634 97.79) (width 0.508) (layer "F.Cu") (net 15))
 (segment (start 104.2466 101.7016) (end 106.685 104.14) (width 0.508) (layer "F.Cu") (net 15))
 (segment (start 44.47488 97.79) (end 48.38648 101.7016) (width 0.508) (layer "F.Cu") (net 15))
 (segment (start 38.095 104.14) (end 38.095 100.718634) (width 0.508) (layer "F.Cu") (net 15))
 (segment (start 48.38648 101.7016) (end 104.2466 101.7016) (width 0.508) (layer "F.Cu") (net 15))
 (via (at 92.71 101.6) (size 0.8) (drill 0.4) (layers "F.Cu" "B.Cu") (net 15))
 (segment (start 91.17 104.14) (end 92.71 104.14) (width 0.508) (layer "B.Cu") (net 15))
 (segment (start 92.71 104.14) (end 92.71 101.6) (width 0.508) (layer "B.Cu") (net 15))
 (segment (start 92.71 104.14) (end 93.98 104.14) (width 0.508) (layer "B.Cu") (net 15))
 (segment (start 190.5 104.14) (end 190.5 102.87) (width 0.508) (layer "F.Cu") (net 18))
 (segment (start 241.3 104.14) (end 182.875 104.14) (width 0.508) (layer "F.Cu") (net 18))
 (via (at 190.5 102.87) (size 0.8) (drill 0.4) (layers "F.Cu" "B.Cu") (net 18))
 (segment (start 190.5 102.87) (end 190.5 104.14) (width 0.508) (layer "B.Cu") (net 18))
 (segment (start 190.5 104.14) (end 188.96 104.14) (width 0.508) (layer "B.Cu") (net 18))
 (segment (start 190.5 104.14) (end 191.77 104.14) (width 0.508) (layer "B.Cu") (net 18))
 (segment (start 212.344 102.362) (end 212.344 101.854) (width 0.5) (layer "F.Cu") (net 19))
 (segment (start 243.84 104.14) (end 241.3 101.6) (width 0.508) (layer "F.Cu") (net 19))
 (segment (start 182.5752 101.9048) (end 182.5702 101.9048) (width 0.508) (layer "F.Cu") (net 19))
 (segment (start 241.3 101.6) (end 212.09 101.6) (width 0.508) (layer "F.Cu") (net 19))
 (segment (start 212.09 101.6) (end 182.88 101.6) (width 0.508) (layer "F.Cu") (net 19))
 (segment (start 212.344 101.854) (end 212.09 101.6) (width 0.5) (layer "F.Cu") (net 19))
 (segment (start 182.5702 101.9048) (end 180.335 104.14) (width 0.508) (layer "F.Cu") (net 19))
 (segment (start 182.88 101.6) (end 182.5752 101.9048) (width 0.508) (layer "F.Cu") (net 19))
 (via (at 212.344 102.362) (size 0.8) (drill 0.4) (layers "F.Cu" "B.Cu") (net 19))
 (segment (start 210.042 104.14) (end 212.344 104.14) (width 0.5) (layer "B.Cu") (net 19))
 (segment (start 212.344 104.14) (end 215.012 104.14) (width 0.5) (layer "B.Cu") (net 19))
 (segment (start 212.344 104.14) (end 212.344 102.362) (width 0.5) (layer "B.Cu") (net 19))
 (segment (start 234.463251 99.399511) (end 235.512283 98.350479) (width 0.5) (layer "F.Cu") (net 20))
 (segment (start 195.961 98.6028) (end 193.458689 96.100489) (width 0.5) (layer "F.Cu") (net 20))
 (segment (start 235.512283 98.350479) (end 242.801101 98.350479) (width 0.5) (layer "F.Cu") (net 20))
 (segment (start 176.53 95.7834) (end 173.99 98.3234) (width 0.5) (layer "F.Cu") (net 20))
 (segment (start 242.801101 98.350479) (end 246.38 101.929378) (width 0.5) (layer "F.Cu") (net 20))
 (segment (start 182.3466 96.9264) (end 181.2036 95.7834) (width 0.5) (layer "F.Cu") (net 20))
 (segment (start 181.2036 95.7834) (end 176.53 95.7834) (width 0.5) (layer "F.Cu") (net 20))
 (segment (start 189.716749 96.100489) (end 188.890838 96.9264) (width 0.5) (layer "F.Cu") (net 20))
 (segment (start 208.5086 93.4974) (end 206.9338 95.0722) (width 0.5) (layer "F.Cu") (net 20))
 (segment (start 222.1484 98.6282) (end 218.4146 94.8944) (width 0.5) (layer "F.Cu") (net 20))
 (segment (start 231.479511 99.399511) (end 234.463251 99.399511) (width 0.5) (layer "F.Cu") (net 20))
 (segment (start 202.1332 98.6028) (end 195.961 98.6028) (width 0.5) (layer "F.Cu") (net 20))
 (segment (start 231.14 99.06) (end 231.479511 99.399511) (width 0.5) (layer "F.Cu") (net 20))
 (segment (start 188.890838 96.9264) (end 182.3466 96.9264) (width 0.5) (layer "F.Cu") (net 20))
 (segment (start 205.6638 95.0722) (end 202.1332 98.6028) (width 0.5) (layer "F.Cu") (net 20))
 (segment (start 218.4146 94.8944) (end 217.2208 94.8944) (width 0.5) (layer "F.Cu") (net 20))
 (segment (start 246.38 101.929378) (end 246.38 104.14) (width 0.5) (layer "F.Cu") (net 20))
 (segment (start 217.2208 94.8944) (end 215.8238 93.4974) (width 0.5) (layer "F.Cu") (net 20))
 (segment (start 193.458689 96.100489) (end 189.716749 96.100489) (width 0.5) (layer "F.Cu") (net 20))
 (segment (start 173.99 98.3234) (end 173.99 100.335) (width 0.5) (layer "F.Cu") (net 20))
 (segment (start 206.9338 95.0722) (end 205.6638 95.0722) (width 0.5) (layer "F.Cu") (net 20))
 (segment (start 215.8238 93.4974) (end 208.5086 93.4974) (width 0.5) (layer "F.Cu") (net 20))
 (segment (start 173.99 100.335) (end 177.795 104.14) (width 0.5) (layer "F.Cu") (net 20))
 (segment (start 230.7082 98.6282) (end 222.1484 98.6282) (width 0.5) (layer "F.Cu") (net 20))
 (segment (start 231.14 99.06) (end 230.7082 98.6282) (width 0.5) (layer "F.Cu") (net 20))
 (via (at 231.14 99.06) (size 0.8) (drill 0.4) (layers "F.Cu" "B.Cu") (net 20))
 (segment (start 231.14 102.041464) (end 231.499469 102.400933) (width 0.508) (layer "B.Cu") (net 20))
 (segment (start 231.499469 104.1146) (end 232.792 104.1146) (width 0.508) (layer "B.Cu") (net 20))
 (segment (start 231.499469 104.1146) (end 231.499469 102.400933) (width 0.508) (layer "B.Cu") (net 20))
 (segment (start 230.235 104.1146) (end 231.499469 104.1146) (width 0.508) (layer "B.Cu") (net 20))
 (segment (start 231.14 99.06) (end 231.14 102.041464) (width 0.508) (layer "B.Cu") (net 20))
 (segment (start 104.14 90.17) (end 76.2 90.17) (width 0.5) (layer "F.Cu") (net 7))
 (segment (start 76.2 90.17) (end 48.26 90.17) (width 0.5) (layer "F.Cu") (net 7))
 (segment (start 104.14 90.17) (end 106.332762 90.17) (width 0.5) (layer "B.Cu") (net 7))
 (segment (start 33.02 91.44) (end 34.29 90.17) (width 1.016) (layer "B.Cu") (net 7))
 (segment (start 33.02 95.222371) (end 33.02 91.44) (width 1.016) (layer "B.Cu") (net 7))
 (segment (start 109.225 93.062238) (end 109.225 104.14) (width 0.5) (layer "B.Cu") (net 7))
 (segment (start 34.29 90.17) (end 48.26 90.17) (width 1.016) (layer "B.Cu") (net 7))
 (segment (start 33.02 101.605) (end 35.555 104.14) (width 1.016) (layer "B.Cu") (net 7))
 (segment (start 106.332762 90.17) (end 109.225 93.062238) (width 0.5) (layer "B.Cu") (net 7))
 (segment (start 33.02 95.222371) (end 33.02 101.605) (width 1.016) (layer "B.Cu") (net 7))
 (segment (start 52.01 91.44) (end 50.7 92.75) (width 0.5) (layer "F.Cu") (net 6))
 (segment (start 92.77 91.44) (end 94.08 92.75) (width 0.5) (layer "F.Cu") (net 6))
 (segment (start 111.765 96.237944) (end 111.765 104.14) (width 0.5) (layer "F.Cu") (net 6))
 (segment (start 94.08 92.75) (end 106.58 92.75) (width 0.5) (layer "F.Cu") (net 6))
 (segment (start 79.95 91.44) (end 92.77 91.44) (width 0.5) (layer "F.Cu") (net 6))
 (segment (start 108.277056 92.75) (end 111.765 96.237944) (width 0.5) (layer "F.Cu") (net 6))
 (segment (start 64.83 91.44) (end 52.01 91.44) (width 0.5) (layer "F.Cu") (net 6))
 (segment (start 66.14 92.75) (end 64.83 91.44) (width 0.5) (layer "F.Cu") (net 6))
 (segment (start 78.64 92.75) (end 79.95 91.44) (width 0.5) (layer "F.Cu") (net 6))
 (segment (start 33.015 97.935) (end 33.015 104.14) (width 0.508) (layer "F.Cu") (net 6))
 (segment (start 106.58 92.75) (end 108.277056 92.75) (width 0.5) (layer "F.Cu") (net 6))
 (segment (start 38.2 92.75) (end 33.015 97.935) (width 0.508) (layer "F.Cu") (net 6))
 (segment (start 66.14 92.75) (end 78.64 92.75) (width 0.5) (layer "F.Cu") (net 6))
 (segment (start 50.7 92.75) (end 38.2 92.75) (width 0.508) (layer "B.Cu") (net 6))
 (segment (start 219.65 91.44) (end 232.47 91.44) (width 0.5) (layer "F.Cu") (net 2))
 (segment (start 218.34 92.75) (end 219.65 91.44) (width 0.5) (layer "F.Cu") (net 2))
 (segment (start 205.84 92.75) (end 218.34 92.75) (width 0.5) (layer "F.Cu") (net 2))
 (segment (start 177.9 92.75) (end 190.4 92.75) (width 0.5) (layer "F.Cu") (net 2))
 (segment (start 172.715 97.935) (end 172.715 104.14) (width 0.5) (layer "F.Cu") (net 2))
 (segment (start 190.4 92.75) (end 191.71 91.44) (width 0.5) (layer "F.Cu") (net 2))
 (segment (start 251.46 97.93) (end 251.46 104.14) (width 0.5) (layer "F.Cu") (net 2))
 (segment (start 204.53 91.44) (end 205.84 92.75) (width 0.5) (layer "F.Cu") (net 2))
 (segment (start 177.9 92.75) (end 172.715 97.935) (width 0.5) (layer "F.Cu") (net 2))
 (segment (start 232.47 91.44) (end 233.78 92.75) (width 0.5) (layer "F.Cu") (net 2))
 (segment (start 233.78 92.75) (end 246.28 92.75) (width 0.5) (layer "F.Cu") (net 2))
 (segment (start 246.28 92.75) (end 251.46 97.93) (width 0.5) (layer "F.Cu") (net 2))
 (segment (start 191.71 91.44) (end 204.53 91.44) (width 0.5) (layer "F.Cu") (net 2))
 (segment (start 187.96 90.17) (end 215.9 90.17) (width 0.5) (layer "F.Cu") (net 3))
 (segment (start 215.9 90.17) (end 243.84 90.17) (width 0.5) (layer "F.Cu") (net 3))
 (segment (start 175.255 97.727762) (end 175.255 104.14) (width 0.5) (layer "B.Cu") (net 3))
 (segment (start 248.915 104.14) (end 248.915 91.435) (width 0.508) (layer "B.Cu") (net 3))
 (segment (start 182.812762 90.17) (end 175.255 97.727762) (width 0.5) (layer "B.Cu") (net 3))
 (segment (start 248.915 91.435) (end 247.65 90.17) (width 0.508) (layer "B.Cu") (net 3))
 (segment (start 247.65 90.17) (end 243.84 90.17) (width 0.508) (layer "B.Cu") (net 3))
 (segment (start 187.96 90.17) (end 182.812762 90.17) (width 0.5) (layer "B.Cu") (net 3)))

